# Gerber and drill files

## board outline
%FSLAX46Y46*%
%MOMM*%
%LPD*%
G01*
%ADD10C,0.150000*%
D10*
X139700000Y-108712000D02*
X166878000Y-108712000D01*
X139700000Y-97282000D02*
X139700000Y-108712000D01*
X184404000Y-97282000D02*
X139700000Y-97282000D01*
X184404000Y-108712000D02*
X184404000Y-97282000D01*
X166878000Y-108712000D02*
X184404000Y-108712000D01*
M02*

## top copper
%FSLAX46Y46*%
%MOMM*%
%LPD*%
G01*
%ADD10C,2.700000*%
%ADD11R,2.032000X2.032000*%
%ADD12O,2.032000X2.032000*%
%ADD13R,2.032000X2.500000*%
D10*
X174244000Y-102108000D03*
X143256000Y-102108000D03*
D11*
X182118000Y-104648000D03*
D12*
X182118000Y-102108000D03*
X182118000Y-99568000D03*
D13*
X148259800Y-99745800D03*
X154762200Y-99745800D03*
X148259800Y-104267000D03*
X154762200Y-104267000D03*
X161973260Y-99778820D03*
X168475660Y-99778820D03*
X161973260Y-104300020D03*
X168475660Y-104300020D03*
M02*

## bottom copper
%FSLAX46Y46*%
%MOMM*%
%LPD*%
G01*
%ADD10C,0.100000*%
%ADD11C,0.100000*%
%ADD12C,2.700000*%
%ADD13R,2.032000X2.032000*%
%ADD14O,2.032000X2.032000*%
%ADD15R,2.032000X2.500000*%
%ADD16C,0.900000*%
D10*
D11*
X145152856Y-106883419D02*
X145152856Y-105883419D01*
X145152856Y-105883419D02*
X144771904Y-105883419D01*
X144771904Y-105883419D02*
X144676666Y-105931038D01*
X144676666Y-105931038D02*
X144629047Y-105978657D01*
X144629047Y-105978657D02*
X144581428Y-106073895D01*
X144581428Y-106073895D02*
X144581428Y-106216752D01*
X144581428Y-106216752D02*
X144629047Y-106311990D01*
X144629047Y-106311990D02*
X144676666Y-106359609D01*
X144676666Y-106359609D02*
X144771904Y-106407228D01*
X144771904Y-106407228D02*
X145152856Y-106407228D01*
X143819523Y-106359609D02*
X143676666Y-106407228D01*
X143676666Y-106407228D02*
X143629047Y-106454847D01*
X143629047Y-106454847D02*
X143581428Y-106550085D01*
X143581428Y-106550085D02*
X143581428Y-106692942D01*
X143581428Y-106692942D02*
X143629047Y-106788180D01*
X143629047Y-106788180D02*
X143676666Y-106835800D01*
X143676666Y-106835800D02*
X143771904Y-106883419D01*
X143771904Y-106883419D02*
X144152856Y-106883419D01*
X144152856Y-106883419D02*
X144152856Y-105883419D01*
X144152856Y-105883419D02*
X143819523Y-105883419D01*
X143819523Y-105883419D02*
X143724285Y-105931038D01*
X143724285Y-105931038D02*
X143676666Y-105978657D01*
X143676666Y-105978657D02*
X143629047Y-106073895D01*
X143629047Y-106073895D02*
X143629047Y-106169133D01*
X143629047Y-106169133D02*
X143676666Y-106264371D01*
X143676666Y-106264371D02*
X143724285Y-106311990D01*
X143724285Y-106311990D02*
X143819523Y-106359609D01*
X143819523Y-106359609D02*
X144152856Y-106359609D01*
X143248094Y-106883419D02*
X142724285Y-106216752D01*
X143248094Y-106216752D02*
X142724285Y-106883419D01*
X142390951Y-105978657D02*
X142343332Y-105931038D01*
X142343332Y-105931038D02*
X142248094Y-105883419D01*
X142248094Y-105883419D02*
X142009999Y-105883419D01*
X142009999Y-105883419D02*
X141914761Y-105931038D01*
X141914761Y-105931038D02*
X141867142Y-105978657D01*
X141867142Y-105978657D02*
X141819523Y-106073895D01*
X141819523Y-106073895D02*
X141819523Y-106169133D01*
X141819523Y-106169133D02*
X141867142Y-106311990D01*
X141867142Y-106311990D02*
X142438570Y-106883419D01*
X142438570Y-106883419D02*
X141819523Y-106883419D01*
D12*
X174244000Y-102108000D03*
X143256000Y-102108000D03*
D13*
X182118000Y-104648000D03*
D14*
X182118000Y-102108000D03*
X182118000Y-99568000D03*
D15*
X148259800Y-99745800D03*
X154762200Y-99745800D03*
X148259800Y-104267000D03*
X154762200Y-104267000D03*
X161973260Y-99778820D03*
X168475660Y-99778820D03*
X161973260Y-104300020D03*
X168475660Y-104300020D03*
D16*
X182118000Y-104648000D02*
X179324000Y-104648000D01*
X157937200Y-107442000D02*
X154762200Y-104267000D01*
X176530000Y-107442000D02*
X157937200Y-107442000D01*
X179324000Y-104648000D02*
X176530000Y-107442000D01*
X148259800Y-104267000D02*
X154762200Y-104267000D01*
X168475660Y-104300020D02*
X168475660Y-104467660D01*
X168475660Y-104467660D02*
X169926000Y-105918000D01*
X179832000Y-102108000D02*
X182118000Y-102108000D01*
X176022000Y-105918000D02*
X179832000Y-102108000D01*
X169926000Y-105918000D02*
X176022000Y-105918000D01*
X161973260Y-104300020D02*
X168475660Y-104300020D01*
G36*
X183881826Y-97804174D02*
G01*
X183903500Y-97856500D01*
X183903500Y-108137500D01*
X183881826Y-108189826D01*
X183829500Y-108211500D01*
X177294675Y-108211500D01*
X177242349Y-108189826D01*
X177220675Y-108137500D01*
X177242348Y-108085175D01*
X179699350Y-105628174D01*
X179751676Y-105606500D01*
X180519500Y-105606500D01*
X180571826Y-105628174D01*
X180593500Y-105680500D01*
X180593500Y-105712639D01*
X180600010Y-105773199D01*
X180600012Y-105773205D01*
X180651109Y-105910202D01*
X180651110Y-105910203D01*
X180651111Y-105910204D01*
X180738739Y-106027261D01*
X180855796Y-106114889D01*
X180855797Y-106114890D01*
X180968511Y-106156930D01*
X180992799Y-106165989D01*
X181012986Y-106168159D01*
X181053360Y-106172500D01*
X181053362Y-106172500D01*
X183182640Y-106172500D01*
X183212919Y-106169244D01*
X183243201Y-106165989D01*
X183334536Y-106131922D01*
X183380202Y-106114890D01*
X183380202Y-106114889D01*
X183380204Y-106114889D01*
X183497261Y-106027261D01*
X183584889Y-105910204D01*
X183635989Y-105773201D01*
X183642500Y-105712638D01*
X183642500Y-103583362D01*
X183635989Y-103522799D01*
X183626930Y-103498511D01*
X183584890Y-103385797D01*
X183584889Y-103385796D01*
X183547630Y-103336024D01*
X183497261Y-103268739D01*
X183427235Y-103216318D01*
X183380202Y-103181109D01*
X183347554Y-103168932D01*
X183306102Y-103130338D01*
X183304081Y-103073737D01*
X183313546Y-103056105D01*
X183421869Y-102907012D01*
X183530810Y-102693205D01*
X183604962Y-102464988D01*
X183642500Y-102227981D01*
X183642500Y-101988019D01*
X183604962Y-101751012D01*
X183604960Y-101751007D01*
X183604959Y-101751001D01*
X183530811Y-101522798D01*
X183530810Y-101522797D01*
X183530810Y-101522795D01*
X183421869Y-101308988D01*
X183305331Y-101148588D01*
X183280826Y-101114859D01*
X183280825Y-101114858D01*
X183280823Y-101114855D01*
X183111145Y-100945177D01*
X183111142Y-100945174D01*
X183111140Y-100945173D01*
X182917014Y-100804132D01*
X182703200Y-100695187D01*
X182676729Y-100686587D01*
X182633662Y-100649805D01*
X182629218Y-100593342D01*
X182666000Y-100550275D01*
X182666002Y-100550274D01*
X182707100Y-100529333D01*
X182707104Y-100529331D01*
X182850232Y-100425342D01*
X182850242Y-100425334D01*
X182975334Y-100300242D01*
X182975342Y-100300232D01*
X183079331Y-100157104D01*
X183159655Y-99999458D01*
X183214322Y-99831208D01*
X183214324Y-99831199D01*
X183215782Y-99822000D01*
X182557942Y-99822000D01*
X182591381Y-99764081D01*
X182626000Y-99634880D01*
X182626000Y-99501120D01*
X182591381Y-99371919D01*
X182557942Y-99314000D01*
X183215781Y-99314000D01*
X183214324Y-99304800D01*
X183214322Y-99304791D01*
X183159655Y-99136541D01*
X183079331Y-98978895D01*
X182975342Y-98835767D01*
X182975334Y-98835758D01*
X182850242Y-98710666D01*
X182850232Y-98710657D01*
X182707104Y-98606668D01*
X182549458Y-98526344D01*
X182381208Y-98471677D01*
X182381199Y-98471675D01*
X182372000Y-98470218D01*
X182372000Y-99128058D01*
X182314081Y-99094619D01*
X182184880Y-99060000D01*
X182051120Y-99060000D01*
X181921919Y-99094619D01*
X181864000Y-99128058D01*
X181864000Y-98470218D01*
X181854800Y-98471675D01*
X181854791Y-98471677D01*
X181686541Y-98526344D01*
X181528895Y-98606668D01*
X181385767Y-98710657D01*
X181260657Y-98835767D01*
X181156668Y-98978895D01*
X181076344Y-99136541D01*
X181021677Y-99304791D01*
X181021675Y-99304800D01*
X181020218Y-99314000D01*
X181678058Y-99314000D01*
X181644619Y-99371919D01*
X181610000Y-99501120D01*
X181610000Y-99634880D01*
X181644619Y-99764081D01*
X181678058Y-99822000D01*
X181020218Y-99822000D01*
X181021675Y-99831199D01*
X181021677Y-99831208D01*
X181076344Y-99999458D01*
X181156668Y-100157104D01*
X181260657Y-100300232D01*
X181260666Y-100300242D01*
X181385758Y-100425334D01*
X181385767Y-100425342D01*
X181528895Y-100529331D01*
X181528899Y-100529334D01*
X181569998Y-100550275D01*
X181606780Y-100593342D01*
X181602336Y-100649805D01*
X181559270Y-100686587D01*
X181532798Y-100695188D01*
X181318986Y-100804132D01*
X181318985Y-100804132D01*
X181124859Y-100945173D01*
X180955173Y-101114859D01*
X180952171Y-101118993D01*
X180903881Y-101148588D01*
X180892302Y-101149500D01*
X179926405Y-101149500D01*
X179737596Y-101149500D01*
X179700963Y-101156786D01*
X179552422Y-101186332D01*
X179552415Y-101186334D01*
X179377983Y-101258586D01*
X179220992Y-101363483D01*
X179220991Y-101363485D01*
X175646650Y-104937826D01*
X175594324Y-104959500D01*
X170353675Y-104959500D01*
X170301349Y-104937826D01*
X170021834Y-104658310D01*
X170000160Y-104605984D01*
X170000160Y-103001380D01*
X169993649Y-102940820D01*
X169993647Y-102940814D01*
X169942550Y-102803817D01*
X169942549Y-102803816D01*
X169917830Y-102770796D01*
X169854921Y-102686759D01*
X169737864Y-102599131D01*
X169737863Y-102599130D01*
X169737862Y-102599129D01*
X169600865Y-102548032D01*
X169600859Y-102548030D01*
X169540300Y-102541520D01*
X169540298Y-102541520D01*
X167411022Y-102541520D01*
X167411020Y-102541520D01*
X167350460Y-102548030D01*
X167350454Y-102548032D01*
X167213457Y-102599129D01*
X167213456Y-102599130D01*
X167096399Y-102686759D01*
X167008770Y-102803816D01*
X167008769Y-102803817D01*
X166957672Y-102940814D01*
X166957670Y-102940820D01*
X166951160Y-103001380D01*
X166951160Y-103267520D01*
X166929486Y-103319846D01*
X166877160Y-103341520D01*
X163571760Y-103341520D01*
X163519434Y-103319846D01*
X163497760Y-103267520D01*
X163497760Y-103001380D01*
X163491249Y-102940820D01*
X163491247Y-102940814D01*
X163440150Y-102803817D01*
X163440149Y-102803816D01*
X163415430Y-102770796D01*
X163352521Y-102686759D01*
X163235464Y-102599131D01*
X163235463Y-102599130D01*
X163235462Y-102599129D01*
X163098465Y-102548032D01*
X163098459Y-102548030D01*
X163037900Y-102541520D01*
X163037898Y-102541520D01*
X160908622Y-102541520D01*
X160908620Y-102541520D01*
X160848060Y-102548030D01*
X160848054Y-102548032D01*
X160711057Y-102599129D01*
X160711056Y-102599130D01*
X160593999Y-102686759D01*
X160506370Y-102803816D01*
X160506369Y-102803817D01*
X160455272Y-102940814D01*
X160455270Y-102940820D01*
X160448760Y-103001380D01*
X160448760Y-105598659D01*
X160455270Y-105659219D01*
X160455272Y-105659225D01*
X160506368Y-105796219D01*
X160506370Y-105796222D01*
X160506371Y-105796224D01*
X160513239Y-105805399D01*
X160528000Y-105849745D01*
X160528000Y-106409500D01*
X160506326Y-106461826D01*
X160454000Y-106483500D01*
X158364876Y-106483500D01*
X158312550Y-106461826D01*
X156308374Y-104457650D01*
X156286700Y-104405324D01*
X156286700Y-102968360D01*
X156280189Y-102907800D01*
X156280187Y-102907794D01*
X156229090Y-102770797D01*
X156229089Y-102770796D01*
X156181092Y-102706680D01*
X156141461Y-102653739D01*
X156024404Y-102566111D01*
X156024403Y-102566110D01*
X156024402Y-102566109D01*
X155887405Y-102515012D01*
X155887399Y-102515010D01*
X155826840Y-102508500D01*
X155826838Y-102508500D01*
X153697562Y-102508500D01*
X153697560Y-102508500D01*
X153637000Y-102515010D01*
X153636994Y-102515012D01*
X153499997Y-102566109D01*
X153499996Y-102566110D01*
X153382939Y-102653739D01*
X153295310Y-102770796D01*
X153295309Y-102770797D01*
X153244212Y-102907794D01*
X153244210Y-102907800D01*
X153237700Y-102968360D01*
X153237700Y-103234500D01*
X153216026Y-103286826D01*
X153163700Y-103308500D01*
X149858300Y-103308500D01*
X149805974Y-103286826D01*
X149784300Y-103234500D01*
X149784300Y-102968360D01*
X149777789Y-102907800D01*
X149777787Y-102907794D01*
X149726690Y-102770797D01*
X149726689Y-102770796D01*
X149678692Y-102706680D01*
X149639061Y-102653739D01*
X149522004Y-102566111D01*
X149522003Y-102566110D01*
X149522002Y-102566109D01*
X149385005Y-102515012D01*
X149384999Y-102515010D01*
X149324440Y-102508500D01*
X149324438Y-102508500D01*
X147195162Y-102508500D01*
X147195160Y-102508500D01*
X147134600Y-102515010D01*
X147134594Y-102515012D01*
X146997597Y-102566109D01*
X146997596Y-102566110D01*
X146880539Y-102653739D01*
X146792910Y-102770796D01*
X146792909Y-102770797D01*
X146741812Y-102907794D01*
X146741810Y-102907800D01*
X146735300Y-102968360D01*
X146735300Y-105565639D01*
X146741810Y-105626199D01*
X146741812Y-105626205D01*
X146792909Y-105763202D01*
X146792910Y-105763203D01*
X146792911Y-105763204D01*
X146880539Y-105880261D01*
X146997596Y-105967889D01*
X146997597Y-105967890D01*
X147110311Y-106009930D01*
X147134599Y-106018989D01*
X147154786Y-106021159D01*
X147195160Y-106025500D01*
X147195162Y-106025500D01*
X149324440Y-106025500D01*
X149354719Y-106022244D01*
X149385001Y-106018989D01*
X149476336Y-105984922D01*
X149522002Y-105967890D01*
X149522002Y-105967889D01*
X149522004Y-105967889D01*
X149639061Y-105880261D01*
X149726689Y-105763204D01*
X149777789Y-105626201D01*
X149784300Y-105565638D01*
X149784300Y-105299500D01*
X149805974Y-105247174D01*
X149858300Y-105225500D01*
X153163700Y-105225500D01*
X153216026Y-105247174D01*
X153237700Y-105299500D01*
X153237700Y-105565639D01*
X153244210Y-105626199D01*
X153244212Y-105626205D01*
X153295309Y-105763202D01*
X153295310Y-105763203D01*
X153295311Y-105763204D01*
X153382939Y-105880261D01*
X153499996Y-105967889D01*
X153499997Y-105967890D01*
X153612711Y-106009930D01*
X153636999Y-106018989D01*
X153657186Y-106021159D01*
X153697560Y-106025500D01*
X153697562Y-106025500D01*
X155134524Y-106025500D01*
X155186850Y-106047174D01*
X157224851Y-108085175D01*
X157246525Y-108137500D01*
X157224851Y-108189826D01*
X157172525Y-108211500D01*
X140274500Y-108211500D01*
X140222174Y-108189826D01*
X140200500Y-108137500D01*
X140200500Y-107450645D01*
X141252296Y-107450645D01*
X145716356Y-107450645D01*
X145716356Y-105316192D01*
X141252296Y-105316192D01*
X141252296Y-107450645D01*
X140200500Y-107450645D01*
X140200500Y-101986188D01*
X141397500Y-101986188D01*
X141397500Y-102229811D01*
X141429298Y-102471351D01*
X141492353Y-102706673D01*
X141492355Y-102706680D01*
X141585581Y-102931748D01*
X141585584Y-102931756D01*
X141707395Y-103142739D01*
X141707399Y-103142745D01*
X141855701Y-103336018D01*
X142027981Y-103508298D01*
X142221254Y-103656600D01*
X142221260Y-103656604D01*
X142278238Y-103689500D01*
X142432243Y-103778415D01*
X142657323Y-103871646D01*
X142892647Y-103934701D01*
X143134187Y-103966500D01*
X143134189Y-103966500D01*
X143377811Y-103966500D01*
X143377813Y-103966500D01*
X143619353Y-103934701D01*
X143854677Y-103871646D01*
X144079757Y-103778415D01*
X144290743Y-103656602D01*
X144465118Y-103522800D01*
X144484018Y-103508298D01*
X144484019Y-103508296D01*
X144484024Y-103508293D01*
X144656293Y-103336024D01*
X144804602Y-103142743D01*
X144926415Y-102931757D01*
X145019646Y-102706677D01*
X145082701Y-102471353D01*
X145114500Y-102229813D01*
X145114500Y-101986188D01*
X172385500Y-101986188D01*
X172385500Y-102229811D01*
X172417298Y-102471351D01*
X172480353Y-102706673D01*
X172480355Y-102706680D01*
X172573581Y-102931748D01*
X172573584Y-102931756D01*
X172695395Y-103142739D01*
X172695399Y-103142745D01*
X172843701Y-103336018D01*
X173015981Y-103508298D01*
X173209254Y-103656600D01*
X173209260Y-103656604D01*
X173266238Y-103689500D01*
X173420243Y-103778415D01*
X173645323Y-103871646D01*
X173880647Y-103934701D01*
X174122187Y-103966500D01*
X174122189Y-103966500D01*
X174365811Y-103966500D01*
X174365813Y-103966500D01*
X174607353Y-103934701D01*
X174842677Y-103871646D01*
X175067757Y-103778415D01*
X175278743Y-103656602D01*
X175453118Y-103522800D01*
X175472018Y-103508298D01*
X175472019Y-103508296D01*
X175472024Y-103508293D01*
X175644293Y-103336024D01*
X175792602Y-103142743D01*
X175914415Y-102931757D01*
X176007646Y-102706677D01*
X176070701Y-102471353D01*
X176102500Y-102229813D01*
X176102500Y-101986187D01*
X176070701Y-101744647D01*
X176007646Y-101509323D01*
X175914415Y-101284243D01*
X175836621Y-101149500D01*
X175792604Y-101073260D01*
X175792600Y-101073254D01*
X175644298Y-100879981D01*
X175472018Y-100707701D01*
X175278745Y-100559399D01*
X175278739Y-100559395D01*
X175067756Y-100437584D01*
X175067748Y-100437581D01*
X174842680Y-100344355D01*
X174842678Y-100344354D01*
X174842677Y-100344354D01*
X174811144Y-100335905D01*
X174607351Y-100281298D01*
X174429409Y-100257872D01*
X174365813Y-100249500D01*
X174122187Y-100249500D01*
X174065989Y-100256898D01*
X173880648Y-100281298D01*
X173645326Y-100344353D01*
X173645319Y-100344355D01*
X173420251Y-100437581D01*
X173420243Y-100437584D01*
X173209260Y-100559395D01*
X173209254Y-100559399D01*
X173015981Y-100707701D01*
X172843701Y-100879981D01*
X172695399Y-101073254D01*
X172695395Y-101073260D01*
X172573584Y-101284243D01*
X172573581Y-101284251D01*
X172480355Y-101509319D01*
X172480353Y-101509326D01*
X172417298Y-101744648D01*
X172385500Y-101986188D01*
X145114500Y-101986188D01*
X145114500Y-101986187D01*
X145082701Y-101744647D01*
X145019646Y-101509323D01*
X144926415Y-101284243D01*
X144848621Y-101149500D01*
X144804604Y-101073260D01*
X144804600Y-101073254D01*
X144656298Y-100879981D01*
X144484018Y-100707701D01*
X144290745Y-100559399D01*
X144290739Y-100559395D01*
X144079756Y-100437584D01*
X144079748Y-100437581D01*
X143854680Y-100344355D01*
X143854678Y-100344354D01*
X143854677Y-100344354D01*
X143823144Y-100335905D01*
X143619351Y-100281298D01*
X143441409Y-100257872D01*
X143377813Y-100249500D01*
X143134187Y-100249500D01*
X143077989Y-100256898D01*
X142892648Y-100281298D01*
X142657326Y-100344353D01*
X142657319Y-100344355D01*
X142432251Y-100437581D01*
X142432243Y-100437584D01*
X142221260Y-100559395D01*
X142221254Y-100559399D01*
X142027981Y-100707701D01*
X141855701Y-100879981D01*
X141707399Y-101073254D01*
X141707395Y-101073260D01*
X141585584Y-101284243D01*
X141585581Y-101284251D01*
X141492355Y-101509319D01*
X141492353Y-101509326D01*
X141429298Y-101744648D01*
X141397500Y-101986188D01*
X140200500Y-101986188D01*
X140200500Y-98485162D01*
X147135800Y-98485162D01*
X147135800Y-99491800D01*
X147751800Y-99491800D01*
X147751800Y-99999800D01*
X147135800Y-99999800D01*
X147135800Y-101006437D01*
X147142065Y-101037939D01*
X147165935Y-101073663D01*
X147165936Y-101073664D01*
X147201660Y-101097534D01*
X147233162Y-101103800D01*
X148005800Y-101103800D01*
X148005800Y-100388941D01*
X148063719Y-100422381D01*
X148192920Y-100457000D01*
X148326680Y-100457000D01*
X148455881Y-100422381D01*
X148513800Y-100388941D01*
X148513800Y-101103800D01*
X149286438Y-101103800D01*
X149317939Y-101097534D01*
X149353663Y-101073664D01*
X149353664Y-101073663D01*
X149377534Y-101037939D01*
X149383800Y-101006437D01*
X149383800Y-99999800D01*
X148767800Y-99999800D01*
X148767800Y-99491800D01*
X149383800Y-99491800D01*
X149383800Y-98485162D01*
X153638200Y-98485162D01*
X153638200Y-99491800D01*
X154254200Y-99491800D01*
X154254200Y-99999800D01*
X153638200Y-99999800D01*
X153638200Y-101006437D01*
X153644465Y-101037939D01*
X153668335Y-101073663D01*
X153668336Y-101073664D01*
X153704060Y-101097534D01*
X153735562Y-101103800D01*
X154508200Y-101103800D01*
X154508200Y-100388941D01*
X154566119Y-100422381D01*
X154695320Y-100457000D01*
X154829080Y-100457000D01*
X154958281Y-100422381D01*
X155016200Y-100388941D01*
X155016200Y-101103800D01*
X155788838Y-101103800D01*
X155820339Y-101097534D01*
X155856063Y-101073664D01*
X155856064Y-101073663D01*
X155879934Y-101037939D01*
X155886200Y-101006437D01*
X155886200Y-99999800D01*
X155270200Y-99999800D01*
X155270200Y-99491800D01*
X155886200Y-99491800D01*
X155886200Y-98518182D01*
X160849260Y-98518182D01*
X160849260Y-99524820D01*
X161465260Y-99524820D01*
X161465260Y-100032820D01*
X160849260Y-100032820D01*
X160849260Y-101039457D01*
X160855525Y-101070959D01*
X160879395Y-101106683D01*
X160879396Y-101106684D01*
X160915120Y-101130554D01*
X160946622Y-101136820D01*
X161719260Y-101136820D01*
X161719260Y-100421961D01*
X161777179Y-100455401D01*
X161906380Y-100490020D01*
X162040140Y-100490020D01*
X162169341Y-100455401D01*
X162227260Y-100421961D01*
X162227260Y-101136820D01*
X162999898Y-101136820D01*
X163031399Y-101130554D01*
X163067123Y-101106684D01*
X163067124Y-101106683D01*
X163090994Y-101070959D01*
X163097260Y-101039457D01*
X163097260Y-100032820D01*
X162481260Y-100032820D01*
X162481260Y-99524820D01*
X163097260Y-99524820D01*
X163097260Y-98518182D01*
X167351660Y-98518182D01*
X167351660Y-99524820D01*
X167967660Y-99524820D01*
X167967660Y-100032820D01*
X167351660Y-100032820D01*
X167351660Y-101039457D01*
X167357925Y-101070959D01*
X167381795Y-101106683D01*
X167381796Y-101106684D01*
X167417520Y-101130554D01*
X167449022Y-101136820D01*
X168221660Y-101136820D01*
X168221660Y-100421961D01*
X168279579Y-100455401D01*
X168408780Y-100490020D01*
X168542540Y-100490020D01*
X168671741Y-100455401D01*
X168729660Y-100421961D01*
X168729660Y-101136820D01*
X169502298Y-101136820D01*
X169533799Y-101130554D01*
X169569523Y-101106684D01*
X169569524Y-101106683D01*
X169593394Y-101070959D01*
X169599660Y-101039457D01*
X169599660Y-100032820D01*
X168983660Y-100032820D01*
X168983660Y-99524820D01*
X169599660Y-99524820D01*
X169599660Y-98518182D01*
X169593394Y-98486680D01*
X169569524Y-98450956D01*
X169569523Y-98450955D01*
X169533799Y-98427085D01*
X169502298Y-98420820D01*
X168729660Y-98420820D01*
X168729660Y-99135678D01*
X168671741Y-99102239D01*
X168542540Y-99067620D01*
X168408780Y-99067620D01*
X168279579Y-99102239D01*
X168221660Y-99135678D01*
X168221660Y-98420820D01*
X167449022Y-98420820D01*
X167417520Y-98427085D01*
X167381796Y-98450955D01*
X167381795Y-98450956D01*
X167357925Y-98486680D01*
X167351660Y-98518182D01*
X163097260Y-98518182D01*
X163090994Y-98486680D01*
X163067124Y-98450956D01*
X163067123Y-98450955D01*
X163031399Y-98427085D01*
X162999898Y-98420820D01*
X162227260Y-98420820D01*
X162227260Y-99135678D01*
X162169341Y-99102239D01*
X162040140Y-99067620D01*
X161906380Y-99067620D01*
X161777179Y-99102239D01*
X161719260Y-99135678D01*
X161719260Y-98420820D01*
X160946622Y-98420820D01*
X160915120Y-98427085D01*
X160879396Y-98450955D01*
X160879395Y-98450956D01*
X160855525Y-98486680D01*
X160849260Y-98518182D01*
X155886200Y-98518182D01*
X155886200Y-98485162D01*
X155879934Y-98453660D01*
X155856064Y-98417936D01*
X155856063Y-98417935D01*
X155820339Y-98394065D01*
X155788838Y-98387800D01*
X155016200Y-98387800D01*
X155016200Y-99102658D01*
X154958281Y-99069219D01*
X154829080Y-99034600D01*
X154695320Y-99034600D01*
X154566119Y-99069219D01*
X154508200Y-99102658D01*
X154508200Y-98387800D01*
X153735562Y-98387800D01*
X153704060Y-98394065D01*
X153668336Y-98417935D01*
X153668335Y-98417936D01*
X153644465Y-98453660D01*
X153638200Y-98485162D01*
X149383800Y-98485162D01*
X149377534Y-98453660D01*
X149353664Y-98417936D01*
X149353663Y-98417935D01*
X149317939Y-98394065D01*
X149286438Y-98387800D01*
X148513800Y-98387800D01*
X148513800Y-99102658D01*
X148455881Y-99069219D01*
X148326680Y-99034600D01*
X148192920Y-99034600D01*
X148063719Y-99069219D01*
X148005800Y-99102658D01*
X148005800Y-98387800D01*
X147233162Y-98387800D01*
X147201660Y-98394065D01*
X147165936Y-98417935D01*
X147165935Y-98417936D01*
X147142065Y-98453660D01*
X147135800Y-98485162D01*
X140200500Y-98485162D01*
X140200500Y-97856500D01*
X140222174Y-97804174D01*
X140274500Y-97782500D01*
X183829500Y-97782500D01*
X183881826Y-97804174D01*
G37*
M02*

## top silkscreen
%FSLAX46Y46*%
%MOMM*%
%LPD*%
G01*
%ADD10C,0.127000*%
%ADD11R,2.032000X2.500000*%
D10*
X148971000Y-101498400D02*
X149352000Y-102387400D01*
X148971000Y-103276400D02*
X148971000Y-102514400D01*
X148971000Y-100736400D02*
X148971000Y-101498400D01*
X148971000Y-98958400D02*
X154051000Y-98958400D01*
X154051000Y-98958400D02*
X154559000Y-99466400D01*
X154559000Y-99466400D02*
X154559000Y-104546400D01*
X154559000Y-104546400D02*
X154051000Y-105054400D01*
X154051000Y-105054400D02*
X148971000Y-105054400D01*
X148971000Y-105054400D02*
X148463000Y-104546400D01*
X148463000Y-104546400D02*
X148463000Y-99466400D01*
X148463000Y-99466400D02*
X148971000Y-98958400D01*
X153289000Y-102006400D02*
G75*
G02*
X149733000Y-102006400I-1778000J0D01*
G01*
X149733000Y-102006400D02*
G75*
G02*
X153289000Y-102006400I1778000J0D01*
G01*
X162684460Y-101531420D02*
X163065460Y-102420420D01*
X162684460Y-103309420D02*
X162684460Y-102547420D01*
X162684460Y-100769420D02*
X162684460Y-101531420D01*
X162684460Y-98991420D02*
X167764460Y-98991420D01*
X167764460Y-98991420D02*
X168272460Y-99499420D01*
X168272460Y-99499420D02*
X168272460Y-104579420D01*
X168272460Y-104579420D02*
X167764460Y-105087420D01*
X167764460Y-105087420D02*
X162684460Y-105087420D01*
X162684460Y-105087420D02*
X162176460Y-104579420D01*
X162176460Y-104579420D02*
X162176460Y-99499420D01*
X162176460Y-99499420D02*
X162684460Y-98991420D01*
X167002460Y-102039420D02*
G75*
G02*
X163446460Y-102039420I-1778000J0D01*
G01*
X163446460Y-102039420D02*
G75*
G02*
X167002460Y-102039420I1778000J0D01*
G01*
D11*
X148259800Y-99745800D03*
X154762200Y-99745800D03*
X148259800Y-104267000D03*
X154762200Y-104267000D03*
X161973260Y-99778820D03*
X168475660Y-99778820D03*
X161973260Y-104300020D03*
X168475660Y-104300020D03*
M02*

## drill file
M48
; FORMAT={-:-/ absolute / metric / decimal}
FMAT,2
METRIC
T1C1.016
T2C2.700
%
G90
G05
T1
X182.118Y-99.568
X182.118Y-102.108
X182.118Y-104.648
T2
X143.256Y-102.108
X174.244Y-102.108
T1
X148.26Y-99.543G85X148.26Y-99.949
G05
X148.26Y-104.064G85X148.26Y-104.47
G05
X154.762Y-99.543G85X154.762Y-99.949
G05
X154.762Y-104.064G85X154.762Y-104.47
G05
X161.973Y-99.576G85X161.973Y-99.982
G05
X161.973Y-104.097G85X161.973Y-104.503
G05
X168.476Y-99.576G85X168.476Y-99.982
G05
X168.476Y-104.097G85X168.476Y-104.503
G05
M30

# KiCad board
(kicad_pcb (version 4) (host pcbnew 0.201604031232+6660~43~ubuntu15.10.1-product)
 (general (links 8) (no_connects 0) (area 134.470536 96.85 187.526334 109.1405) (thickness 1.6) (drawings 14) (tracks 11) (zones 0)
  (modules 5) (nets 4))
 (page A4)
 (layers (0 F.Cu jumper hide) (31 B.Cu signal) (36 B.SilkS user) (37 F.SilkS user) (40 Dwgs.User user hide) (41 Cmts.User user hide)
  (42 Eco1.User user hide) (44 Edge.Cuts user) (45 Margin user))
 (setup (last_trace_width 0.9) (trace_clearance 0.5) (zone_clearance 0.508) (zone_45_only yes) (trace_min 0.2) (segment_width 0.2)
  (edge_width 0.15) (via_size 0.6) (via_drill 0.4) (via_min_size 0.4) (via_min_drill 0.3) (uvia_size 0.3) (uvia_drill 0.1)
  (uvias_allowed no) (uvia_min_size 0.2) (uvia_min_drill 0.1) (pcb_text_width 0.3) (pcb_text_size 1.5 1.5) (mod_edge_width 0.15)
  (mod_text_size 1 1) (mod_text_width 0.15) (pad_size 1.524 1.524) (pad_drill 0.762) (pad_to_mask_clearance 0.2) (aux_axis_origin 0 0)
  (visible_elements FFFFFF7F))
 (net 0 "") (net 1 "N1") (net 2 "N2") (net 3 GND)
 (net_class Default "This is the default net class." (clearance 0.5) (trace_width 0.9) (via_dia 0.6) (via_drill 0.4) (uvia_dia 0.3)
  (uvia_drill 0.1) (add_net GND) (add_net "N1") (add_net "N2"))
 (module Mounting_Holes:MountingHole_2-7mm (layer F.Cu) (at 174.244 102.108)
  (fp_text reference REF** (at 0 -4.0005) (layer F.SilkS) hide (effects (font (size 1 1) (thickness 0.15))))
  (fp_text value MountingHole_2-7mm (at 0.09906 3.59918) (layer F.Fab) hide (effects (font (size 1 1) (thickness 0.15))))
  (pad 1 thru_hole circle (at 0 0) (size 2.7 2.7) (drill 2.7) (layers)))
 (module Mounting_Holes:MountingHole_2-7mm (layer F.Cu) (at 143.256 102.108)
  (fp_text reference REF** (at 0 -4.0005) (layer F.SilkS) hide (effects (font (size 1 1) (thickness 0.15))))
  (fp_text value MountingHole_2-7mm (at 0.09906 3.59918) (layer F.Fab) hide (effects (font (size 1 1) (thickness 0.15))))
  (pad 1 thru_hole circle (at 0 0) (size 2.7 2.7) (drill 2.7) (layers)))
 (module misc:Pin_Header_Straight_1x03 (layer B.Cu) (at 182.118 104.648)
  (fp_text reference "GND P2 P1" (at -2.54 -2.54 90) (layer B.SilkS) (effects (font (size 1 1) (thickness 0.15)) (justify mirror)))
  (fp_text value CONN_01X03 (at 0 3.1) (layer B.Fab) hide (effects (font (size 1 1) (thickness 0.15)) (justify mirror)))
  (pad 1 thru_hole rect (at 0 0) (size 2.032 2.032) (drill 1.016) (layers *.Cu *.Mask B.SilkS) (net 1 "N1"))
  (pad 2 thru_hole oval (at 0 -2.54) (size 2.032 2.032) (drill 1.016) (layers *.Cu *.Mask B.SilkS) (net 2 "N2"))
  (pad 3 thru_hole oval (at 0 -5.08) (size 2.032 2.032) (drill 1.016) (layers *.Cu *.Mask B.SilkS) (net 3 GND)))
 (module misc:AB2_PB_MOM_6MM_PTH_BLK (layer F.Cu) (at 151.511 102.0064)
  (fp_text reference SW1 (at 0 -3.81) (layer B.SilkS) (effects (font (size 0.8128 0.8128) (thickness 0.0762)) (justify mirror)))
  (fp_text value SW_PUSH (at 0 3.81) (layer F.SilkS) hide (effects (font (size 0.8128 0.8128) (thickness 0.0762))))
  (fp_line (start -2.54 -0.508) (end -2.159 0.381) (layer F.SilkS) (width 0.127))
  (fp_line (start -2.54 1.27) (end -2.54 0.508) (layer F.SilkS) (width 0.127))
  (fp_line (start -2.54 -1.27) (end -2.54 -0.508) (layer F.SilkS) (width 0.127))
  (fp_line (start -2.54 -3.048) (end 2.54 -3.048) (layer F.SilkS) (width 0.127))
  (fp_line (start 2.54 -3.048) (end 3.048 -2.54) (layer F.SilkS) (width 0.127))
  (fp_line (start 3.048 -2.54) (end 3.048 2.54) (layer F.SilkS) (width 0.127))
  (fp_line (start 3.048 2.54) (end 2.54 3.048) (layer F.SilkS) (width 0.127))
  (fp_line (start 2.54 3.048) (end -2.54 3.048) (layer F.SilkS) (width 0.127))
  (fp_line (start -2.54 3.048) (end -3.048 2.54) (layer F.SilkS) (width 0.127))
  (fp_line (start -3.048 2.54) (end -3.048 -2.54) (layer F.SilkS) (width 0.127))
  (fp_line (start -3.048 -2.54) (end -2.54 -3.048) (layer F.SilkS) (width 0.127))
  (fp_circle (center 0 0) (end 0 -1.778) (layer F.SilkS) (width 0.127))
  (pad 1 thru_hole rect (at -3.2512 -2.2606) (size 2.032 2.5) (drill oval 1.016 1.4224) (layers *.Cu *.Mask F.SilkS) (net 3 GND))
  (pad 1 thru_hole rect (at 3.2512 -2.2606) (size 2.032 2.5) (drill oval 1.016 1.4224) (layers *.Cu *.Mask F.SilkS) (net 3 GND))
  (pad 2 thru_hole rect (at -3.2512 2.2606) (size 2.032 2.5) (drill oval 1.016 1.4224) (layers *.Cu *.Mask F.SilkS) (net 1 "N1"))
  (pad 2 thru_hole rect (at 3.2512 2.2606) (size 2.032 2.5) (drill oval 1.016 1.4224) (layers *.Cu *.Mask F.SilkS) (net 1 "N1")))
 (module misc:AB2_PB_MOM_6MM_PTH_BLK (layer F.Cu) (at 165.22446 102.03942)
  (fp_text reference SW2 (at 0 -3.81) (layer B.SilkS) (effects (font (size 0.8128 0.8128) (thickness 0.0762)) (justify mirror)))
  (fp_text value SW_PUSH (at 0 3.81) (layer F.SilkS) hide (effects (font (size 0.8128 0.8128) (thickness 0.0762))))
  (fp_line (start -2.54 -0.508) (end -2.159 0.381) (layer F.SilkS) (width 0.127))
  (fp_line (start -2.54 1.27) (end -2.54 0.508) (layer F.SilkS) (width 0.127))
  (fp_line (start -2.54 -1.27) (end -2.54 -0.508) (layer F.SilkS) (width 0.127))
  (fp_line (start -2.54 -3.048) (end 2.54 -3.048) (layer F.SilkS) (width 0.127))
  (fp_line (start 2.54 -3.048) (end 3.048 -2.54) (layer F.SilkS) (width 0.127))
  (fp_line (start 3.048 -2.54) (end 3.048 2.54) (layer F.SilkS) (width 0.127))
  (fp_line (start 3.048 2.54) (end 2.54 3.048) (layer F.SilkS) (width 0.127))
  (fp_line (start 2.54 3.048) (end -2.54 3.048) (layer F.SilkS) (width 0.127))
  (fp_line (start -2.54 3.048) (end -3.048 2.54) (layer F.SilkS) (width 0.127))
  (fp_line (start -3.048 2.54) (end -3.048 -2.54) (layer F.SilkS) (width 0.127))
  (fp_line (start -3.048 -2.54) (end -2.54 -3.048) (layer F.SilkS) (width 0.127))
  (fp_circle (center 0 0) (end 0 -1.778) (layer F.SilkS) (width 0.127))
  (pad 1 thru_hole rect (at -3.2512 -2.2606) (size 2.032 2.5) (drill oval 1.016 1.4224) (layers *.Cu *.Mask F.SilkS) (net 3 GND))
  (pad 1 thru_hole rect (at 3.2512 -2.2606) (size 2.032 2.5) (drill oval 1.016 1.4224) (layers *.Cu *.Mask F.SilkS) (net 3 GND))
  (pad 2 thru_hole rect (at -3.2512 2.2606) (size 2.032 2.5) (drill oval 1.016 1.4224) (layers *.Cu *.Mask F.SilkS) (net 2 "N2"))
  (pad 2 thru_hole rect (at 3.2512 2.2606) (size 2.032 2.5) (drill oval 1.016 1.4224) (layers *.Cu *.Mask F.SilkS) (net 2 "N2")))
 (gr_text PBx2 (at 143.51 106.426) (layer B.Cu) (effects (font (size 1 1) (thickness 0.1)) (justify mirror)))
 (gr_line (start 139.7 108.712) (end 166.878 108.712) (angle 90) (layer Edge.Cuts) (width 0.15))
 (gr_line (start 139.7 97.282) (end 139.7 108.712) (angle 90) (layer Edge.Cuts) (width 0.15))
 (gr_line (start 184.404 97.282) (end 139.7 97.282) (angle 90) (layer Edge.Cuts) (width 0.15))
 (gr_line (start 184.404 108.712) (end 184.404 97.282) (angle 90) (layer Edge.Cuts) (width 0.15))
 (gr_line (start 166.878 108.712) (end 184.404 108.712) (angle 90) (layer Edge.Cuts) (width 0.15))
 (segment (start 182.118 104.648) (end 179.324 104.648) (width 0.9) (layer B.Cu) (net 1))
 (segment (start 157.9372 107.442) (end 154.7622 104.267) (width 0.9) (layer B.Cu) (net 1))
 (segment (start 176.53 107.442) (end 157.9372 107.442) (width 0.9) (layer B.Cu) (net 1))
 (segment (start 179.324 104.648) (end 176.53 107.442) (width 0.9) (layer B.Cu) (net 1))
 (segment (start 148.2598 104.267) (end 154.7622 104.267) (width 0.9) (layer B.Cu) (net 1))
 (segment (start 168.47566 104.30002) (end 168.47566 104.46766) (width 0.9) (layer B.Cu) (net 2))
 (segment (start 168.47566 104.46766) (end 169.926 105.918) (width 0.9) (layer B.Cu) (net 2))
 (segment (start 179.832 102.108) (end 182.118 102.108) (width 0.9) (layer B.Cu) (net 2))
 (segment (start 176.022 105.918) (end 179.832 102.108) (width 0.9) (layer B.Cu) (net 2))
 (segment (start 169.926 105.918) (end 176.022 105.918) (width 0.9) (layer B.Cu) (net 2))
 (segment (start 161.97326 104.30002) (end 168.47566 104.30002) (width 0.9) (layer B.Cu) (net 2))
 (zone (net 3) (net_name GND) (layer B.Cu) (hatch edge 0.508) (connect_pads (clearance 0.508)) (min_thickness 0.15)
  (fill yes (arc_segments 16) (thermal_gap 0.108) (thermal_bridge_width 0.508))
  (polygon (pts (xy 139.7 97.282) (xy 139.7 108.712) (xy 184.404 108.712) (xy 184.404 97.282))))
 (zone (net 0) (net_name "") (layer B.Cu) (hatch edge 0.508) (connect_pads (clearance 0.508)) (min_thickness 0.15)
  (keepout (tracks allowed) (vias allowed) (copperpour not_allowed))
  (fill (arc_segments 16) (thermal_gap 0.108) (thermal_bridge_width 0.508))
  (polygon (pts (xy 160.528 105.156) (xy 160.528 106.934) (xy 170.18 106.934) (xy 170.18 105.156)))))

